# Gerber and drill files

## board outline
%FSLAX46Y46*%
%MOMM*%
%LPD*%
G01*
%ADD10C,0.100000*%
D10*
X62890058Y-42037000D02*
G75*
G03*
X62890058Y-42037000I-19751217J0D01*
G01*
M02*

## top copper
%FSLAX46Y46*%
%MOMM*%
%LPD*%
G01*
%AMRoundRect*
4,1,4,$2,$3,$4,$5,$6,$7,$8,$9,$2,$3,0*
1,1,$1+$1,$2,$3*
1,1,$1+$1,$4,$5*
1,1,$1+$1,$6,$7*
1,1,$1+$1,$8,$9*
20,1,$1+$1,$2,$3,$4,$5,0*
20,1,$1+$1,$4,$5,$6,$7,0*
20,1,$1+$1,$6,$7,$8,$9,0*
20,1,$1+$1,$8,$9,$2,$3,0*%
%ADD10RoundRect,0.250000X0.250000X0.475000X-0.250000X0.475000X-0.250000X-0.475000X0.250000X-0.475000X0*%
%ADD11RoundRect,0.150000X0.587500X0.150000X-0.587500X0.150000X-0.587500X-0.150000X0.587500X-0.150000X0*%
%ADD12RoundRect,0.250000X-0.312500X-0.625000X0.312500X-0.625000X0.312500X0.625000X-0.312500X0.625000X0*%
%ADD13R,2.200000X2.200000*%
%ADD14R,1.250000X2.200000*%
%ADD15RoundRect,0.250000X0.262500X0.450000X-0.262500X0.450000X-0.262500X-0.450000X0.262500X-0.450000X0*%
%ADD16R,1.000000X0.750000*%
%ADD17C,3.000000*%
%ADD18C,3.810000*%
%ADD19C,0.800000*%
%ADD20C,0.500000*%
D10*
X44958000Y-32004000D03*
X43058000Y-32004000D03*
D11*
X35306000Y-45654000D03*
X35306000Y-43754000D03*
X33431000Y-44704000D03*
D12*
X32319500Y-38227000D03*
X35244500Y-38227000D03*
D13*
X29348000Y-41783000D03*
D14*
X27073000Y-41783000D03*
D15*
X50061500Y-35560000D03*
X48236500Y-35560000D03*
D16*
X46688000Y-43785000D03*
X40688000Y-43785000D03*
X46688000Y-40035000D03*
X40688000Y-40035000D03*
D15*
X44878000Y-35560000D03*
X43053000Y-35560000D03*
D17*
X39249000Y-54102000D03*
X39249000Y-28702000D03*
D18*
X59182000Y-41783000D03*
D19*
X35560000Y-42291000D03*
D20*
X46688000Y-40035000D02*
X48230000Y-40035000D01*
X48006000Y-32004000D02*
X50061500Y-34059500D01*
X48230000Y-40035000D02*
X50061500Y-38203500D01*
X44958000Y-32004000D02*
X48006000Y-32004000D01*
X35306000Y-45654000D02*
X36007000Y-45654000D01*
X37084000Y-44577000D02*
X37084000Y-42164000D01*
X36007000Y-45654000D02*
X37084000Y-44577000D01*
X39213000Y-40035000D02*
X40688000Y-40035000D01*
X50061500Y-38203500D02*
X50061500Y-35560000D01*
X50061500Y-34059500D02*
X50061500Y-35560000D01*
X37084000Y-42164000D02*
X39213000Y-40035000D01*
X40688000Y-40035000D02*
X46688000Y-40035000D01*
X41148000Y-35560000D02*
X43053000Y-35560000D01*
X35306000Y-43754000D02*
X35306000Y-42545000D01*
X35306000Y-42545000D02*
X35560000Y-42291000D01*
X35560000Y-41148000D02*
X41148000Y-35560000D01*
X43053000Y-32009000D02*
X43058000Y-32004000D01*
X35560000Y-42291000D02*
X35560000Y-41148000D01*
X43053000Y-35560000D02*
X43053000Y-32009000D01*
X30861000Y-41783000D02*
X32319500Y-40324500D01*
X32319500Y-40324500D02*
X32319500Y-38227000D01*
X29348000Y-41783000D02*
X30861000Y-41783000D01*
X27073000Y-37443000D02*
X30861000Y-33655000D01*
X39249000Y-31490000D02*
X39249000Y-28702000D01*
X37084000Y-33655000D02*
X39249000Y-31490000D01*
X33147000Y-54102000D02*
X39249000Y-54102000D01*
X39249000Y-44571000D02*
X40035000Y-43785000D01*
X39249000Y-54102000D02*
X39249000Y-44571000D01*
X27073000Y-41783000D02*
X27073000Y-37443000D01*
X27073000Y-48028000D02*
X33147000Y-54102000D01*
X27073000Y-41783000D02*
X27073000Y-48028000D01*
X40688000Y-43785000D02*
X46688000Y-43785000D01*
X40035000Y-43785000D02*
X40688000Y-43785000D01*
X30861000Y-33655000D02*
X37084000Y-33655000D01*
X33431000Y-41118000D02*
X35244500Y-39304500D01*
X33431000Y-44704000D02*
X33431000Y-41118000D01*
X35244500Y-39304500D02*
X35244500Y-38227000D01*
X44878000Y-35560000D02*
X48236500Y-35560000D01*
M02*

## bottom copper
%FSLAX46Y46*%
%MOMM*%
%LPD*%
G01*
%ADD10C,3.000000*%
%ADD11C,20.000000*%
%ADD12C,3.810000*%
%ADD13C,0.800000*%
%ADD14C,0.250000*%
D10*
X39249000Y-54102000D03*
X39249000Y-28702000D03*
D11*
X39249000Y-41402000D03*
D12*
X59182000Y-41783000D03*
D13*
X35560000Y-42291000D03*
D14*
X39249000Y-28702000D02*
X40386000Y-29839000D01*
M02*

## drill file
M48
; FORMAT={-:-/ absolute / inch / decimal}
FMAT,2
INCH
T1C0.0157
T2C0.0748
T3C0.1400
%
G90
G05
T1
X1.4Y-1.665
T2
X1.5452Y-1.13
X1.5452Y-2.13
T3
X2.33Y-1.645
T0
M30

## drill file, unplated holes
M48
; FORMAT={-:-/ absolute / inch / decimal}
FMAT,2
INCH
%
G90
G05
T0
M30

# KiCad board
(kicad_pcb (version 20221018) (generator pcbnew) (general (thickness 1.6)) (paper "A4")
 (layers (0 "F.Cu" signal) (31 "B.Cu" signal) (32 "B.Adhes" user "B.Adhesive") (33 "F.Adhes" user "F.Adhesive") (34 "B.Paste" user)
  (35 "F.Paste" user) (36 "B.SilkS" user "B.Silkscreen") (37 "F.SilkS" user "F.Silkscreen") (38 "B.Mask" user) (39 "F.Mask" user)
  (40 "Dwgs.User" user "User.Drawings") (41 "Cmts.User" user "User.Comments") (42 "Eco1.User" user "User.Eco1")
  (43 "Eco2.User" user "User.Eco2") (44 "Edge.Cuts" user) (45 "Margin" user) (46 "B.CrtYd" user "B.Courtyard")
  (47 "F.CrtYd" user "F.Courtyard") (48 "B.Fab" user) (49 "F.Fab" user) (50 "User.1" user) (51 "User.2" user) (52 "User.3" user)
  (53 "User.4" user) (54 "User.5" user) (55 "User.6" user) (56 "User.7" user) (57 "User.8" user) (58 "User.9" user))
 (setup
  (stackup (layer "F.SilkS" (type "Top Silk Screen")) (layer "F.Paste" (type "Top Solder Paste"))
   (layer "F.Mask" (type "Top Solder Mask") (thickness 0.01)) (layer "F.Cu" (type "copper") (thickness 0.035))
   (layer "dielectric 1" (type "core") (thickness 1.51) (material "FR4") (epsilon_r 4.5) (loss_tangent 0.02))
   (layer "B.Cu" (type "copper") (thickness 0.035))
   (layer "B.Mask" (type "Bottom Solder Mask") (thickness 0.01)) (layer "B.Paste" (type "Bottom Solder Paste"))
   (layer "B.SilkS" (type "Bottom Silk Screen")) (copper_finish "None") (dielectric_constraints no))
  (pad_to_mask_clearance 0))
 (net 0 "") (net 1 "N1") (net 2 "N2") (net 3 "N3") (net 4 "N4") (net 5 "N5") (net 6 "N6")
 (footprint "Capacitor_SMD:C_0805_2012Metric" (layer "F.Cu") (at 44.008 32.004 180)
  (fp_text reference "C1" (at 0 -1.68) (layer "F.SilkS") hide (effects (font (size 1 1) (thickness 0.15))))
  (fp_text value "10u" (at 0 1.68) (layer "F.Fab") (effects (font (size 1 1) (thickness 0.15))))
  (pad "1" smd roundrect (at -0.95 0 180) (size 1 1.45) (layers "F.Cu" "F.Paste" "F.Mask") (roundrect_rratio 0.25) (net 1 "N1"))
  (pad "2" smd roundrect (at 0.95 0 180) (size 1 1.45) (layers "F.Cu" "F.Paste" "F.Mask") (roundrect_rratio 0.25) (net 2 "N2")))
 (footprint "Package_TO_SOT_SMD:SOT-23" (layer "F.Cu") (at 34.3685 44.704 180)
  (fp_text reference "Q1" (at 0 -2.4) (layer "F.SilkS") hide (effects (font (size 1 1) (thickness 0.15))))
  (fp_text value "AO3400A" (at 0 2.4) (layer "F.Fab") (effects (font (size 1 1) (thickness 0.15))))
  (pad "1" smd roundrect (at -0.9375 -0.95 180) (size 1.475 0.6) (layers "F.Cu" "F.Paste" "F.Mask") (roundrect_rratio 0.25) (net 1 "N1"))
  (pad "2" smd roundrect (at -0.9375 0.95 180) (size 1.475 0.6) (layers "F.Cu" "F.Paste" "F.Mask") (roundrect_rratio 0.25) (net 2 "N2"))
  (pad "3" smd roundrect (at 0.9375 0 180) (size 1.475 0.6) (layers "F.Cu" "F.Paste" "F.Mask") (roundrect_rratio 0.25) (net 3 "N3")))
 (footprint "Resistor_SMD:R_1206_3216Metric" (layer "F.Cu") (at 33.782 38.227)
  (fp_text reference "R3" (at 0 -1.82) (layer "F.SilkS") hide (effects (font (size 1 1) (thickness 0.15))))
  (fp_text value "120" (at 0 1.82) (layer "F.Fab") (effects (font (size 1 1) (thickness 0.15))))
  (pad "1" smd roundrect (at -1.4625 0) (size 1.125 1.75) (layers "F.Cu" "F.Paste" "F.Mask") (roundrect_rratio 0.2222222222) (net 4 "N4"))
  (pad "2" smd roundrect (at 1.4625 0) (size 1.125 1.75) (layers "F.Cu" "F.Paste" "F.Mask") (roundrect_rratio 0.2222222222) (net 3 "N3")))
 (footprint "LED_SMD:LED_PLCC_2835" (layer "F.Cu") (at 28.448 41.783 180)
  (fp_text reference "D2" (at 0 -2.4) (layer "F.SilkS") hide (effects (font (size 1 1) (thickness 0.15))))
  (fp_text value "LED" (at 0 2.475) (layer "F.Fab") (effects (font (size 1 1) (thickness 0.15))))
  (pad "1" smd rect (at -0.9 0 180) (size 2.2 2.2) (layers "F.Cu" "F.Paste" "F.Mask") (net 4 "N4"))
  (pad "2" smd rect (at 1.375 0 180) (size 1.25 2.2) (layers "F.Cu" "F.Paste" "F.Mask") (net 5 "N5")))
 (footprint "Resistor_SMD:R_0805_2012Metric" (layer "F.Cu") (at 49.149 35.56 180)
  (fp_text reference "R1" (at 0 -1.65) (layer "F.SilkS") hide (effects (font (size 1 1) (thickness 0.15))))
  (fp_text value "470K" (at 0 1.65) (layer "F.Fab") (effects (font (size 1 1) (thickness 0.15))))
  (pad "1" smd roundrect (at -0.9125 0 180) (size 1.025 1.4) (layers "F.Cu" "F.Paste" "F.Mask") (roundrect_rratio 0.243902439) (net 1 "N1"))
  (pad "2" smd roundrect (at 0.9125 0 180) (size 1.025 1.4) (layers "F.Cu" "F.Paste" "F.Mask") (roundrect_rratio 0.243902439) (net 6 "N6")))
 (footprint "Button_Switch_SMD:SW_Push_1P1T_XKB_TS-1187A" (layer "F.Cu") (at 43.688 41.91 180)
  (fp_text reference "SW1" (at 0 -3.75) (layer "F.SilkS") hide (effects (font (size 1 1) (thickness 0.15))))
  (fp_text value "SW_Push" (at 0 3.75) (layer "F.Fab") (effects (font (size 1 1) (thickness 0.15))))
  (pad "1" smd rect (at -3 -1.875 180) (size 1 0.75) (layers "F.Cu" "F.Paste" "F.Mask") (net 5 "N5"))
  (pad "1" smd rect (at 3 -1.875 180) (size 1 0.75) (layers "F.Cu" "F.Paste" "F.Mask") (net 5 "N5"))
  (pad "2" smd rect (at -3 1.875 180) (size 1 0.75) (layers "F.Cu" "F.Paste" "F.Mask") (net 1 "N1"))
  (pad "2" smd rect (at 3 1.875 180) (size 1 0.75) (layers "F.Cu" "F.Paste" "F.Mask") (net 1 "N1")))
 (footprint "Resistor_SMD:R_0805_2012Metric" (layer "F.Cu") (at 43.9655 35.56 180)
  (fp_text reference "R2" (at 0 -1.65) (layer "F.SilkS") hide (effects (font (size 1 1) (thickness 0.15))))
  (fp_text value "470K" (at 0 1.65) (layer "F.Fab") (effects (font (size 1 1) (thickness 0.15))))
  (pad "1" smd roundrect (at -0.9125 0 180) (size 1.025 1.4) (layers "F.Cu" "F.Paste" "F.Mask") (roundrect_rratio 0.243902439) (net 6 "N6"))
  (pad "2" smd roundrect (at 0.9125 0 180) (size 1.025 1.4) (layers "F.Cu" "F.Paste" "F.Mask") (roundrect_rratio 0.243902439) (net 2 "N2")))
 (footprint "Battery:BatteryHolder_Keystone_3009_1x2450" (layer "B.Cu") (at 39.249 41.402 90)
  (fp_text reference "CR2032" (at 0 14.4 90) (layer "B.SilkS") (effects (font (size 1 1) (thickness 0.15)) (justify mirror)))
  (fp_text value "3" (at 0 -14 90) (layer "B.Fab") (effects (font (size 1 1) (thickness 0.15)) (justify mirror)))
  (pad "1" thru_hole circle (at -12.7 0 90) (size 3 3) (drill 1.9) (layers "*.Cu" "*.Mask") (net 5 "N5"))
  (pad "1" thru_hole circle (at 12.7 0 90) (size 3 3) (drill 1.9) (layers "*.Cu" "*.Mask") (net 5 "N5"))
  (pad "2" smd circle (at 0 0 90) (size 20 20) (layers "B.Cu" "B.Mask") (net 2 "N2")))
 (gr_circle (center 43.138841 42.037) (end 60.579 51.308) (stroke (width 0.1) (type default)) (fill none) (layer "Edge.Cuts"))
 (via (at 59.182 41.783) (size 3.81) (drill 3.556) (layers "F.Cu" "B.Cu") (free) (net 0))
 (segment (start 46.688 40.035) (end 48.23 40.035) (width 0.5) (layer "F.Cu") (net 1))
 (segment (start 48.006 32.004) (end 50.0615 34.0595) (width 0.5) (layer "F.Cu") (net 1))
 (segment (start 48.23 40.035) (end 50.0615 38.2035) (width 0.5) (layer "F.Cu") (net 1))
 (segment (start 44.958 32.004) (end 48.006 32.004) (width 0.5) (layer "F.Cu") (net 1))
 (segment (start 35.306 45.654) (end 36.007 45.654) (width 0.5) (layer "F.Cu") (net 1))
 (segment (start 37.084 44.577) (end 37.084 42.164) (width 0.5) (layer "F.Cu") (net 1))
 (segment (start 36.007 45.654) (end 37.084 44.577) (width 0.5) (layer "F.Cu") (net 1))
 (segment (start 39.213 40.035) (end 40.688 40.035) (width 0.5) (layer "F.Cu") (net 1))
 (segment (start 50.0615 38.2035) (end 50.0615 35.56) (width 0.5) (layer "F.Cu") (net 1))
 (segment (start 50.0615 34.0595) (end 50.0615 35.56) (width 0.5) (layer "F.Cu") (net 1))
 (segment (start 37.084 42.164) (end 39.213 40.035) (width 0.5) (layer "F.Cu") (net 1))
 (segment (start 40.688 40.035) (end 46.688 40.035) (width 0.5) (layer "F.Cu") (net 1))
 (segment (start 41.148 35.56) (end 43.053 35.56) (width 0.5) (layer "F.Cu") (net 2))
 (segment (start 35.306 43.754) (end 35.306 42.545) (width 0.5) (layer "F.Cu") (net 2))
 (segment (start 35.306 42.545) (end 35.56 42.291) (width 0.5) (layer "F.Cu") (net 2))
 (segment (start 35.56 41.148) (end 41.148 35.56) (width 0.5) (layer "F.Cu") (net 2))
 (segment (start 43.053 32.009) (end 43.058 32.004) (width 0.5) (layer "F.Cu") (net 2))
 (segment (start 35.56 42.291) (end 35.56 41.148) (width 0.5) (layer "F.Cu") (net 2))
 (segment (start 43.053 35.56) (end 43.053 32.009) (width 0.5) (layer "F.Cu") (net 2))
 (via (at 35.56 42.291) (size 0.8) (drill 0.4) (layers "F.Cu" "B.Cu") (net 2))
 (segment (start 30.861 41.783) (end 32.3195 40.3245) (width 0.5) (layer "F.Cu") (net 4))
 (segment (start 32.3195 40.3245) (end 32.3195 38.227) (width 0.5) (layer "F.Cu") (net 4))
 (segment (start 29.348 41.783) (end 30.861 41.783) (width 0.5) (layer "F.Cu") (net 4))
 (segment (start 27.073 37.443) (end 30.861 33.655) (width 0.5) (layer "F.Cu") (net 5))
 (segment (start 39.249 31.49) (end 39.249 28.702) (width 0.5) (layer "F.Cu") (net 5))
 (segment (start 37.084 33.655) (end 39.249 31.49) (width 0.5) (layer "F.Cu") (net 5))
 (segment (start 33.147 54.102) (end 39.249 54.102) (width 0.5) (layer "F.Cu") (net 5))
 (segment (start 39.249 44.571) (end 40.035 43.785) (width 0.5) (layer "F.Cu") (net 5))
 (segment (start 39.249 54.102) (end 39.249 44.571) (width 0.5) (layer "F.Cu") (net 5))
 (segment (start 27.073 41.783) (end 27.073 37.443) (width 0.5) (layer "F.Cu") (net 5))
 (segment (start 27.073 48.028) (end 33.147 54.102) (width 0.5) (layer "F.Cu") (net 5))
 (segment (start 27.073 41.783) (end 27.073 48.028) (width 0.5) (layer "F.Cu") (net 5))
 (segment (start 40.688 43.785) (end 46.688 43.785) (width 0.5) (layer "F.Cu") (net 5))
 (segment (start 40.035 43.785) (end 40.688 43.785) (width 0.5) (layer "F.Cu") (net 5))
 (segment (start 30.861 33.655) (end 37.084 33.655) (width 0.5) (layer "F.Cu") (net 5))
 (segment (start 39.249 28.702) (end 40.386 29.839) (width 0.25) (layer "B.Cu") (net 5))
 (segment (start 33.431 41.118) (end 35.2445 39.3045) (width 0.5) (layer "F.Cu") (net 3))
 (segment (start 33.431 44.704) (end 33.431 41.118) (width 0.5) (layer "F.Cu") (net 3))
 (segment (start 35.2445 39.3045) (end 35.2445 38.227) (width 0.5) (layer "F.Cu") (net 3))
 (segment (start 44.878 35.56) (end 48.2365 35.56) (width 0.5) (layer "F.Cu") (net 6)))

